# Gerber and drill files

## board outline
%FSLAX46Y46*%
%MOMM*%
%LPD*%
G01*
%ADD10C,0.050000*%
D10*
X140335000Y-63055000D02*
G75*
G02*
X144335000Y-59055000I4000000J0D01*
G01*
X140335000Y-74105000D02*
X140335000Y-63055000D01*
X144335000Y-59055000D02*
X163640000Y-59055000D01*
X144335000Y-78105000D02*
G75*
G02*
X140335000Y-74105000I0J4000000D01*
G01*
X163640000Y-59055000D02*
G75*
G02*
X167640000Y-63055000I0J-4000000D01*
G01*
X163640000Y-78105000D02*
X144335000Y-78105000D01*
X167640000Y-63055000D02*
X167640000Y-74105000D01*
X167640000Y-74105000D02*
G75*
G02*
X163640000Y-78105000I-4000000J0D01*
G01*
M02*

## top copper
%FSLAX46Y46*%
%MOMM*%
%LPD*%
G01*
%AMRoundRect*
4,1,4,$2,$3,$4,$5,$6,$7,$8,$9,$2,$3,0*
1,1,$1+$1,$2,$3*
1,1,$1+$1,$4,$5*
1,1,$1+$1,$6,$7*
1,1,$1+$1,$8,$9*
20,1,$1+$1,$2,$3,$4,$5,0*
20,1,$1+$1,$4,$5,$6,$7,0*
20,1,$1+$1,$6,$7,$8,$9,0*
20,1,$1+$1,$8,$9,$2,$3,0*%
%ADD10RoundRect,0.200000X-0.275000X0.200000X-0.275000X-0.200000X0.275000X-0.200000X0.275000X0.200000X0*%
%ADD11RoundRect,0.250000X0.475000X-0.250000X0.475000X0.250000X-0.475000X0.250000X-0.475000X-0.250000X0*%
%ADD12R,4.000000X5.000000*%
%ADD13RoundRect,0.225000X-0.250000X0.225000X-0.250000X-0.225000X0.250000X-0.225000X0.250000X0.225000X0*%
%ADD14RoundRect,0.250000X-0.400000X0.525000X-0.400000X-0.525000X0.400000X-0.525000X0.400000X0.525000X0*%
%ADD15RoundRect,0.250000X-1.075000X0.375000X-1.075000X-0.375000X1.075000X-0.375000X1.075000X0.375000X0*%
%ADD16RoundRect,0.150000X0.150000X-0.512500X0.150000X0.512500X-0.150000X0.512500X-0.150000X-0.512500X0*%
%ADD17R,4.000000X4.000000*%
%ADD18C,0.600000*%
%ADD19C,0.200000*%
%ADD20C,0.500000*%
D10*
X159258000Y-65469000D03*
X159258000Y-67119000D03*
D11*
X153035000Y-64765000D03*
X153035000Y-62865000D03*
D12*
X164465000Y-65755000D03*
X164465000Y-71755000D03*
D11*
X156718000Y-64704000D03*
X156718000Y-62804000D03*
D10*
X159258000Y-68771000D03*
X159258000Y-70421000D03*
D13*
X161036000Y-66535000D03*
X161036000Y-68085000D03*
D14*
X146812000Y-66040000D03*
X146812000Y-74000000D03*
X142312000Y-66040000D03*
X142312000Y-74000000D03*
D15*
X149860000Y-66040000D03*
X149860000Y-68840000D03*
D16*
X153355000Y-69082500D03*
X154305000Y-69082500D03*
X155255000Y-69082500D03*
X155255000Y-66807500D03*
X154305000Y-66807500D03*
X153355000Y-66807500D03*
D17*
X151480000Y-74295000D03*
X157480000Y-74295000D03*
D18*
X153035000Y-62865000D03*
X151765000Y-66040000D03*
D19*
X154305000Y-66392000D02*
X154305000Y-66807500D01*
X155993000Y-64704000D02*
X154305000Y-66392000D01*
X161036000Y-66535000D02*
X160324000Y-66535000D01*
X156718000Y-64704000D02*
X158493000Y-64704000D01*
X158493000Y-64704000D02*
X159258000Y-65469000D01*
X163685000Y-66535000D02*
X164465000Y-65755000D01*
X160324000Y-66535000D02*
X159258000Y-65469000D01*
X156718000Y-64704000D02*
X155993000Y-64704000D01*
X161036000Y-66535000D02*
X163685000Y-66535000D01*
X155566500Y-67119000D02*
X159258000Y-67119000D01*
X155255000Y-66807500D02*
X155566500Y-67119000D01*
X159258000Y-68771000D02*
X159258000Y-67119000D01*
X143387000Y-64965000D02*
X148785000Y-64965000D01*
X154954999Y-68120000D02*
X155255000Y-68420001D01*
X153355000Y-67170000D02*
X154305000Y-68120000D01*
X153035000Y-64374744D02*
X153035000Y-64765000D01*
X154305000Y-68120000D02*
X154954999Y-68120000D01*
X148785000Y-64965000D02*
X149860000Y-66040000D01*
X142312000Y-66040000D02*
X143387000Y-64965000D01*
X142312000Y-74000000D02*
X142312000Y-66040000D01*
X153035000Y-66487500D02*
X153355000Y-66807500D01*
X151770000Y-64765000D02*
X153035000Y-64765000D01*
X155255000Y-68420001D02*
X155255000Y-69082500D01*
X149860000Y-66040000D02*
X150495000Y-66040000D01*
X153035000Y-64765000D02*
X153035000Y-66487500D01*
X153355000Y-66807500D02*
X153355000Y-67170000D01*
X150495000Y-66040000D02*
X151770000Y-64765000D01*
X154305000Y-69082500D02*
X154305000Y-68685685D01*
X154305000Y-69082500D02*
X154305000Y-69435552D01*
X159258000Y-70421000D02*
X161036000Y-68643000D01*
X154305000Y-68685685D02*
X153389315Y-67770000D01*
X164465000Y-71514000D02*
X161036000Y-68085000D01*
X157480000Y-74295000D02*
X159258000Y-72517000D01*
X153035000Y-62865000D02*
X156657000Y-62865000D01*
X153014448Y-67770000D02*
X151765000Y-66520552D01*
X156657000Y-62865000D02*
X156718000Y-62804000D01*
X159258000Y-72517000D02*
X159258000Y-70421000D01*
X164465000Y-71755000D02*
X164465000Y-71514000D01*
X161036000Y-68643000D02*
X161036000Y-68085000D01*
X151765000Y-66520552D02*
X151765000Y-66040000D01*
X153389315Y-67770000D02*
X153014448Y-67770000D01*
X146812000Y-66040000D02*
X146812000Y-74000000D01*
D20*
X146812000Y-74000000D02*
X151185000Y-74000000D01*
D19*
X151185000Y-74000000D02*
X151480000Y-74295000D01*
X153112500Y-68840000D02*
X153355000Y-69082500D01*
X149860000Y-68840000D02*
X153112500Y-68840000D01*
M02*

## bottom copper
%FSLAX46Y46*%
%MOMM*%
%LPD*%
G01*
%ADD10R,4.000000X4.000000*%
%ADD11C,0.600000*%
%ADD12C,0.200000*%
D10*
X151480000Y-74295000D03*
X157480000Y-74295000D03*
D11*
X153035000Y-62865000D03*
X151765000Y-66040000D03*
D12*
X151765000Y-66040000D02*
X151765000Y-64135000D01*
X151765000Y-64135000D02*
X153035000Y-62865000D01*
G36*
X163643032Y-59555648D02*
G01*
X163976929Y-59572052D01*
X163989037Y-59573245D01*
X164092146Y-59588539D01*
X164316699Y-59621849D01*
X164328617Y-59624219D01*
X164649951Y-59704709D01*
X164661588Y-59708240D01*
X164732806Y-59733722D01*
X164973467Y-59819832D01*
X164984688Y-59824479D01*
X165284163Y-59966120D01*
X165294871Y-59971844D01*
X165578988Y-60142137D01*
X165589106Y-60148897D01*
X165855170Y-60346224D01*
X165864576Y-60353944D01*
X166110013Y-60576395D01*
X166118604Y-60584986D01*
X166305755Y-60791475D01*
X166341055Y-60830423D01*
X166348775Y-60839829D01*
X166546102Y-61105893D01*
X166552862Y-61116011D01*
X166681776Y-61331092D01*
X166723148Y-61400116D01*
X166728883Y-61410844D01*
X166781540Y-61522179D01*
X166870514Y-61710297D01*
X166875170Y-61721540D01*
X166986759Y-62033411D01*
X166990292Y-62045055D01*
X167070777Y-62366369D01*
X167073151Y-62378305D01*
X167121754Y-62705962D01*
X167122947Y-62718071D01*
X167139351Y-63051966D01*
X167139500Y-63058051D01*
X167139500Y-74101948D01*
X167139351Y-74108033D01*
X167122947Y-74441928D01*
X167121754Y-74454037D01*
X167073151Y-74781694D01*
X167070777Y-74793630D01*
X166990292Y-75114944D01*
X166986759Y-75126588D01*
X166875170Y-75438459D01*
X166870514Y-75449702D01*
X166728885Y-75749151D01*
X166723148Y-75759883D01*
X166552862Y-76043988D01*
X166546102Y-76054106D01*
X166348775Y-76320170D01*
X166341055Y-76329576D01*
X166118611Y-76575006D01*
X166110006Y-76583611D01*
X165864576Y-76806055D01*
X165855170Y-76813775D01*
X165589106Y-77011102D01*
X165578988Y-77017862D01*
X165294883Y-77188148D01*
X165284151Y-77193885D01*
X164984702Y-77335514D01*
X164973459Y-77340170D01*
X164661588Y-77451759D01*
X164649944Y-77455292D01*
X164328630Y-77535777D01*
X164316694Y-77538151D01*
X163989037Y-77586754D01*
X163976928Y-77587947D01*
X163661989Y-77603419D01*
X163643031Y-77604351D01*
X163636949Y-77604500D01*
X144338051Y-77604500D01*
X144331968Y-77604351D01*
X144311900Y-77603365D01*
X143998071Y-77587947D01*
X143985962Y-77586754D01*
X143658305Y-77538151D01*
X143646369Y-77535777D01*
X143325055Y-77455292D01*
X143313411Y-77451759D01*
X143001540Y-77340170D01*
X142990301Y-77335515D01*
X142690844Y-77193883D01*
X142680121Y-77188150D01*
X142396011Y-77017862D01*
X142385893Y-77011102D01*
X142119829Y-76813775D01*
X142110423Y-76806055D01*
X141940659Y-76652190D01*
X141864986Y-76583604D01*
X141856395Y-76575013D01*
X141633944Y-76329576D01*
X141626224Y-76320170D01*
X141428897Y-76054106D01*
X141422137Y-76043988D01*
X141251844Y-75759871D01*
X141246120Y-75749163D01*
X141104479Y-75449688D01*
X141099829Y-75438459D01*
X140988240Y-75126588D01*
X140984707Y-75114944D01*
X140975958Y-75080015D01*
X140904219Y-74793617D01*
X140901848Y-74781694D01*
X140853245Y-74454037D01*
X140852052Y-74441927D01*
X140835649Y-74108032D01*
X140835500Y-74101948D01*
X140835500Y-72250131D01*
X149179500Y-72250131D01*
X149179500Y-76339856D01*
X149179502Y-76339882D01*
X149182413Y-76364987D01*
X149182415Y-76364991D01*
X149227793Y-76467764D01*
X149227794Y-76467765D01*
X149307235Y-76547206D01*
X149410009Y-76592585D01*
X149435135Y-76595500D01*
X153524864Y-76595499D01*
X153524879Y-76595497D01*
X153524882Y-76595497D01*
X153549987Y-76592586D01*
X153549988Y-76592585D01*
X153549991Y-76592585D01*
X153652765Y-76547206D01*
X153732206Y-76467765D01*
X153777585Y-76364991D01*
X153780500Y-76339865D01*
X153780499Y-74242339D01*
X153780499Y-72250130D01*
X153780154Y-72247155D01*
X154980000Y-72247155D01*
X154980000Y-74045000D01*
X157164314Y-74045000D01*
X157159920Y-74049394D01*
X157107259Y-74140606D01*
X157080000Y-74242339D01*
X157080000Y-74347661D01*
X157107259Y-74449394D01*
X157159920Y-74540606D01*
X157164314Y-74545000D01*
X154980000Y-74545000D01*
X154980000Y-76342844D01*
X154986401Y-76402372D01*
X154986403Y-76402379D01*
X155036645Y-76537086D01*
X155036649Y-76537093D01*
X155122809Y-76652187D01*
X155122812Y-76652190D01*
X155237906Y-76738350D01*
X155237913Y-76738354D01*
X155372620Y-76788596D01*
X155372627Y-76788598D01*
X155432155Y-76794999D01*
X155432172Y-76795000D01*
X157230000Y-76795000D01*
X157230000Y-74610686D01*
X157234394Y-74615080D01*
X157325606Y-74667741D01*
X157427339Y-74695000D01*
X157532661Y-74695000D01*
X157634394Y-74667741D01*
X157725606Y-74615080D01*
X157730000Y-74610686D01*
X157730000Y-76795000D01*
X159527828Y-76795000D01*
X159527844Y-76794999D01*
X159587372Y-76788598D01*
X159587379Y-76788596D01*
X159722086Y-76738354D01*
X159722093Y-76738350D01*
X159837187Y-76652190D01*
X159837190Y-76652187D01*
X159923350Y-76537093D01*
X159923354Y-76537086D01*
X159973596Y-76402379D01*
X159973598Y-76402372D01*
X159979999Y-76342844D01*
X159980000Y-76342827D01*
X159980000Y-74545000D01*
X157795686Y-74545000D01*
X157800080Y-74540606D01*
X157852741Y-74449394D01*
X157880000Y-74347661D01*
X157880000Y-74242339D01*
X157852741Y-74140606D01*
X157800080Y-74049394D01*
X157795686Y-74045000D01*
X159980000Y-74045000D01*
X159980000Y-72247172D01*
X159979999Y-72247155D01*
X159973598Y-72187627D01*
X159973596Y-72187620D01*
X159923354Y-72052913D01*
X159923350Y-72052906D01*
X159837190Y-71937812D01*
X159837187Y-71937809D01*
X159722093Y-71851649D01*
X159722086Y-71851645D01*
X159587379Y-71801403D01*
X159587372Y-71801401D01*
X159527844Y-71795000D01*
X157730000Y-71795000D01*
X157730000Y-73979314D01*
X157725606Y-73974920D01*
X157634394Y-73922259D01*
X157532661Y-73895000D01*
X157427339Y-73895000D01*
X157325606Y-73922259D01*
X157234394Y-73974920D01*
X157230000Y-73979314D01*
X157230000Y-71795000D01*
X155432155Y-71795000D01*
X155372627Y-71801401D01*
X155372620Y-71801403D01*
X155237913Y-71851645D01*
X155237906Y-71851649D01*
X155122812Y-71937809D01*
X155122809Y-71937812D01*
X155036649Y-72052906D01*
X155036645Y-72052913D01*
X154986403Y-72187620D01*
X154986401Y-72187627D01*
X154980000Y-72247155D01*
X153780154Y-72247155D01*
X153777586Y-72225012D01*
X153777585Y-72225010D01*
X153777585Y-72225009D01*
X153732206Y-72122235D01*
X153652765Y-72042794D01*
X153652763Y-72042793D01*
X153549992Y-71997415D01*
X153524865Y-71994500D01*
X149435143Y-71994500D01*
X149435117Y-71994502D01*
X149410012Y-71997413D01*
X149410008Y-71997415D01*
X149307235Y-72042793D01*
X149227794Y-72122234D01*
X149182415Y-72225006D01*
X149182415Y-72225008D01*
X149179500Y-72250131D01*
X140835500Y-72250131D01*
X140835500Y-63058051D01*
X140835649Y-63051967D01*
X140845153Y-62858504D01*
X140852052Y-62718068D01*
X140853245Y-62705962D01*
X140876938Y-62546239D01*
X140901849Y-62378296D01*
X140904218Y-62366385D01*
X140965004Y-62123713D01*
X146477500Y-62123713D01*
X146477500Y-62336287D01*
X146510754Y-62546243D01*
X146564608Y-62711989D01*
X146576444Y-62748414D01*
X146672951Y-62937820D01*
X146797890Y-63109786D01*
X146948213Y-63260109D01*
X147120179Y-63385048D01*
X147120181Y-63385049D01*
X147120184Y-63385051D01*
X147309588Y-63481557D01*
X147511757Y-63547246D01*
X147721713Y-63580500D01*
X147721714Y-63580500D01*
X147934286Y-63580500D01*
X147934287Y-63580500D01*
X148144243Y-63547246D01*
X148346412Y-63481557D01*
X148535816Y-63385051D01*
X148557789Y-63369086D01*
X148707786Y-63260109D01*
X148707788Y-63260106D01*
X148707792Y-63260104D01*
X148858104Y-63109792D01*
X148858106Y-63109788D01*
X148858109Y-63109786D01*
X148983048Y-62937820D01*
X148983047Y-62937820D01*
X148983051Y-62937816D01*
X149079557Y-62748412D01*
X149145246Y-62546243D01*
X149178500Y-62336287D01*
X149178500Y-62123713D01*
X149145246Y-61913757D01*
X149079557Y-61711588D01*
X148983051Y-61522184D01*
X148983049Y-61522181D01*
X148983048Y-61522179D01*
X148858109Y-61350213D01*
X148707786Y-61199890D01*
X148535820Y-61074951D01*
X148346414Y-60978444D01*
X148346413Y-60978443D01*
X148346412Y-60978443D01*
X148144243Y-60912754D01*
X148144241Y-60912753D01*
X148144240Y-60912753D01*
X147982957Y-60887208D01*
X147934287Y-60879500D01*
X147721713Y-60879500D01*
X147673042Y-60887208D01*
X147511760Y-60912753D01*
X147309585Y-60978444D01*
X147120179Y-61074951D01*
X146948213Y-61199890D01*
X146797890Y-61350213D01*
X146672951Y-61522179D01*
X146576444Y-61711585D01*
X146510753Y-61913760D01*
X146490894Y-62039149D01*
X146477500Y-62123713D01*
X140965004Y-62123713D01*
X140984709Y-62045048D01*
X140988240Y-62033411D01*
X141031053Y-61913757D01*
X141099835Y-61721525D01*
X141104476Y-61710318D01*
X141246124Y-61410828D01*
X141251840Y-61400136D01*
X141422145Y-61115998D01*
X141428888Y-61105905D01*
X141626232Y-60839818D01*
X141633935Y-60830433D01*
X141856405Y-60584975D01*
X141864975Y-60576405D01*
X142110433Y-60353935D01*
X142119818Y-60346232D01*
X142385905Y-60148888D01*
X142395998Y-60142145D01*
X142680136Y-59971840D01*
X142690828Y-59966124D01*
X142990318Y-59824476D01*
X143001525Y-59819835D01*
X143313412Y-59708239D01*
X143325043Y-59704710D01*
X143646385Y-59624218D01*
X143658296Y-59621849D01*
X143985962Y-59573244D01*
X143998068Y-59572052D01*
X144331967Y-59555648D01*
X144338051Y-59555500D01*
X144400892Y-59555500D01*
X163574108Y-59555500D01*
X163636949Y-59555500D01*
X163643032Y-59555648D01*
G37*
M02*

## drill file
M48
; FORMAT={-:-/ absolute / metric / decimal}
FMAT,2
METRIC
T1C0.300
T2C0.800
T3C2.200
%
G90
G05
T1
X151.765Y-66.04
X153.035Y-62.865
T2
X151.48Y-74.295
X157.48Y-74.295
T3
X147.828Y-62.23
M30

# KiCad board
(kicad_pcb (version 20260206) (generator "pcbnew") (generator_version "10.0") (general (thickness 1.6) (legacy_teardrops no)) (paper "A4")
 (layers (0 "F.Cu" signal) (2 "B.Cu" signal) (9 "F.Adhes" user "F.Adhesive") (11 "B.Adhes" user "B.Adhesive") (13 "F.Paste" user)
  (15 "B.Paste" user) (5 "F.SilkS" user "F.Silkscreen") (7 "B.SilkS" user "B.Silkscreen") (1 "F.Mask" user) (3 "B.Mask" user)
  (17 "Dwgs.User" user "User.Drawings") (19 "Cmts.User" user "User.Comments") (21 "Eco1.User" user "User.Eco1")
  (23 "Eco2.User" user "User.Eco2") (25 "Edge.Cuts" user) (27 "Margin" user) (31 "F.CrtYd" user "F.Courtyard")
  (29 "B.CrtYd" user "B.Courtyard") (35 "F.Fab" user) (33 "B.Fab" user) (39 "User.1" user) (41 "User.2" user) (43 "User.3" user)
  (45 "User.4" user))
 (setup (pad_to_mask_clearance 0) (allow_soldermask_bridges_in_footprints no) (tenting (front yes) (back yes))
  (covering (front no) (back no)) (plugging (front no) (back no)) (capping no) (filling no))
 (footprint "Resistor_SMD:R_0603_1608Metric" (layer "F.Cu") (at 159.258 66.294 -90)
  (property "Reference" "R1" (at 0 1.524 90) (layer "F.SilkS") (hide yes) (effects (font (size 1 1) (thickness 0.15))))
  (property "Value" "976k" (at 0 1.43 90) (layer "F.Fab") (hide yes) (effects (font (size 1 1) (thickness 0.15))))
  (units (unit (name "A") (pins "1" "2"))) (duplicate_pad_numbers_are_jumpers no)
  (pad "1" smd roundrect (at -0.825 0 270) (size 0.8 0.95) (layers "F.Cu" "F.Mask" "F.Paste") (roundrect_rratio 0.25) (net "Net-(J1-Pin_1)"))
  (pad "2" smd roundrect (at 0.825 0 270) (size 0.8 0.95) (layers "F.Cu" "F.Mask" "F.Paste") (roundrect_rratio 0.25) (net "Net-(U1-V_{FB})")))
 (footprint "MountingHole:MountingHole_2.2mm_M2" (layer "F.Cu") (at 147.828 62.23)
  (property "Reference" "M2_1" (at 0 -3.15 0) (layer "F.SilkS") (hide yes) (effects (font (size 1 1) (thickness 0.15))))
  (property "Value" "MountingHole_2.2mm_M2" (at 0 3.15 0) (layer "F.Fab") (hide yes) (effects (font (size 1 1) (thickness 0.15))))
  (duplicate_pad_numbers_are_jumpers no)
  (pad "" np_thru_hole circle (at 0 0) (size 2.2 2.2) (drill 2.2) (layers "*.Cu" "*.Mask")))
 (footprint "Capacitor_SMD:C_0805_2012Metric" (layer "F.Cu") (at 153.035 63.815 90)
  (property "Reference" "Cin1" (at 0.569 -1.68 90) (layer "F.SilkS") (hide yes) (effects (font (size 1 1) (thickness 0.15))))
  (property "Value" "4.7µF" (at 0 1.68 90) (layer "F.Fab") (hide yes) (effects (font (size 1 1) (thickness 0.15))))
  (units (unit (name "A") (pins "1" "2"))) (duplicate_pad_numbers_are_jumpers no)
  (pad "1" smd roundrect (at -0.95 0 90) (size 1 1.45) (layers "F.Cu" "F.Mask" "F.Paste") (roundrect_rratio 0.25) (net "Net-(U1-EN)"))
  (pad "2" smd roundrect (at 0.95 0 90) (size 1 1.45) (layers "F.Cu" "F.Mask" "F.Paste") (roundrect_rratio 0.25) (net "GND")))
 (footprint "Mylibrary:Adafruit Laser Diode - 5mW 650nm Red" (layer "F.Cu") (at 164.465 68.755 -90)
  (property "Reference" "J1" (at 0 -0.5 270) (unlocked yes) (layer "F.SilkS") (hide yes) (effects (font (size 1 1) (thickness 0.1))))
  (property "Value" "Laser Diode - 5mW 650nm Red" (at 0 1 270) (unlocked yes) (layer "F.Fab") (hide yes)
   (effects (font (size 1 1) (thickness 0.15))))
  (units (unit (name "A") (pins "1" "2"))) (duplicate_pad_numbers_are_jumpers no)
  (pad "1" smd rect (at -3 0 270) (size 5 4) (layers "F.Cu" "F.Mask" "F.Paste") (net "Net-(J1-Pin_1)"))
  (pad "2" smd rect (at 3 0 270) (size 5 4) (layers "F.Cu" "F.Mask" "F.Paste") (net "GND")))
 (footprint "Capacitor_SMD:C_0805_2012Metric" (layer "F.Cu") (at 156.718 63.754 90)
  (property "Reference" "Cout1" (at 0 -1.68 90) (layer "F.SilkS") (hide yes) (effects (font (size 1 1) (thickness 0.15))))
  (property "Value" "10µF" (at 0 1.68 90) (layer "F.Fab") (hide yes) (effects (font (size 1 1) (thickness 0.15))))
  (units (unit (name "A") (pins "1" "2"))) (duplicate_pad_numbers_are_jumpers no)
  (pad "1" smd roundrect (at -0.95 0 90) (size 1 1.45) (layers "F.Cu" "F.Mask" "F.Paste") (roundrect_rratio 0.25) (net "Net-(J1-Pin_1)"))
  (pad "2" smd roundrect (at 0.95 0 90) (size 1 1.45) (layers "F.Cu" "F.Mask" "F.Paste") (roundrect_rratio 0.25) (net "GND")))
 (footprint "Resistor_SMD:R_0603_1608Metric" (layer "F.Cu") (at 159.258 69.596 -90)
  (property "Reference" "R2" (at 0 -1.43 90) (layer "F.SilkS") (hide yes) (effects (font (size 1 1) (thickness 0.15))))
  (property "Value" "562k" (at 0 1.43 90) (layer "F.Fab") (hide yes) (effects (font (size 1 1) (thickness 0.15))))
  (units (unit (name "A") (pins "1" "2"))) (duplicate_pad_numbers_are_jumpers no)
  (pad "1" smd roundrect (at -0.825 0 270) (size 0.8 0.95) (layers "F.Cu" "F.Mask" "F.Paste") (roundrect_rratio 0.25)
   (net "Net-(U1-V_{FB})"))
  (pad "2" smd roundrect (at 0.825 0 270) (size 0.8 0.95) (layers "F.Cu" "F.Mask" "F.Paste") (roundrect_rratio 0.25) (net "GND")))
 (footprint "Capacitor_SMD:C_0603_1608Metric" (layer "F.Cu") (at 161.036 67.31 -90)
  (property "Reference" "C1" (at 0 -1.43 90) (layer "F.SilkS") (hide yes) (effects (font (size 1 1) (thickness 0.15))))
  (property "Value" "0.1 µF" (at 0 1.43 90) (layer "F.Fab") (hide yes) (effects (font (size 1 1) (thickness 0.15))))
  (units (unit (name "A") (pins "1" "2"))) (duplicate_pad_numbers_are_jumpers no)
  (pad "1" smd roundrect (at -0.775 0 270) (size 0.9 0.95) (layers "F.Cu" "F.Mask" "F.Paste") (roundrect_rratio 0.25) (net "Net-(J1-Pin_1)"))
  (pad "2" smd roundrect (at 0.775 0 270) (size 0.9 0.95) (layers "F.Cu" "F.Mask" "F.Paste") (roundrect_rratio 0.25) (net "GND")))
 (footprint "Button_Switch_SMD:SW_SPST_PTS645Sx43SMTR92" (layer "F.Cu") (at 144.562 70.02 -90)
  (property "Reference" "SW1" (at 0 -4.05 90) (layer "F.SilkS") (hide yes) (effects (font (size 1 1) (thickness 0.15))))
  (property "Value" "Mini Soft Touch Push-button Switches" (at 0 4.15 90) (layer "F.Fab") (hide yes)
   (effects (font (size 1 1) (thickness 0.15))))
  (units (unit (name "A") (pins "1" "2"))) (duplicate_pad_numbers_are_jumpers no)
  (pad "1" smd roundrect (at -3.98 -2.25 270) (size 1.55 1.3) (layers "F.Cu" "F.Mask" "F.Paste") (roundrect_rratio 0.1923076923)
   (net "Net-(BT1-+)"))
  (pad "1" smd roundrect (at 3.98 -2.25 270) (size 1.55 1.3) (layers "F.Cu" "F.Mask" "F.Paste") (roundrect_rratio 0.1923076923)
   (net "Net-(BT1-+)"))
  (pad "2" smd roundrect (at -3.98 2.25 270) (size 1.55 1.3) (layers "F.Cu" "F.Mask" "F.Paste") (roundrect_rratio 0.1923076923)
   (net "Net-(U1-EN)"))
  (pad "2" smd roundrect (at 3.98 2.25 270) (size 1.55 1.3) (layers "F.Cu" "F.Mask" "F.Paste") (roundrect_rratio 0.1923076923)
   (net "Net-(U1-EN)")))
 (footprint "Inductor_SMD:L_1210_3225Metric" (layer "F.Cu") (at 149.86 67.44 -90)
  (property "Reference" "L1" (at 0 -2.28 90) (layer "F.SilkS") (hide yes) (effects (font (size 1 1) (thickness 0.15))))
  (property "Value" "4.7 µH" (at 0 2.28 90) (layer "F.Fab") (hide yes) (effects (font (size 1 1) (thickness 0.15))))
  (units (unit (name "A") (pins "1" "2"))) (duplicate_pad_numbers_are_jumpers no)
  (pad "1" smd roundrect (at -1.4 0 270) (size 1.25 2.65) (layers "F.Cu" "F.Mask" "F.Paste") (roundrect_rratio 0.2) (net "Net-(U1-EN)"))
  (pad "2" smd roundrect (at 1.4 0 270) (size 1.25 2.65) (layers "F.Cu" "F.Mask" "F.Paste") (roundrect_rratio 0.2) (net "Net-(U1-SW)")))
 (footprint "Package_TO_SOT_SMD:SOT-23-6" (layer "F.Cu") (at 154.305 67.945 90)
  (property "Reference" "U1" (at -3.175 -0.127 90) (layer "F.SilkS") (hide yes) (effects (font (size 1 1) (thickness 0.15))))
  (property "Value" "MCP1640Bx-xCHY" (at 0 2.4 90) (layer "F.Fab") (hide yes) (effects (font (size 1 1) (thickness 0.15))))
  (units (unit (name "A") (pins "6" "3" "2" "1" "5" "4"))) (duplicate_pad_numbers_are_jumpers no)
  (pad "1" smd roundrect (at -1.1375 -0.95 90) (size 1.325 0.6) (layers "F.Cu" "F.Mask" "F.Paste") (roundrect_rratio 0.25)
   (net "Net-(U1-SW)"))
  (pad "2" smd roundrect (at -1.1375 0 90) (size 1.325 0.6) (layers "F.Cu" "F.Mask" "F.Paste") (roundrect_rratio 0.25) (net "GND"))
  (pad "3" smd roundrect (at -1.1375 0.95 90) (size 1.325 0.6) (layers "F.Cu" "F.Mask" "F.Paste") (roundrect_rratio 0.25)
   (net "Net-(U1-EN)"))
  (pad "4" smd roundrect (at 1.1375 0.95 90) (size 1.325 0.6) (layers "F.Cu" "F.Mask" "F.Paste") (roundrect_rratio 0.25)
   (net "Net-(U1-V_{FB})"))
  (pad "5" smd roundrect (at 1.1375 0 90) (size 1.325 0.6) (layers "F.Cu" "F.Mask" "F.Paste") (roundrect_rratio 0.25) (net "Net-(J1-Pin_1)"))
  (pad "6" smd roundrect (at 1.1375 -0.95 90) (size 1.325 0.6) (layers "F.Cu" "F.Mask" "F.Paste") (roundrect_rratio 0.25)
   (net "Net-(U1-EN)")))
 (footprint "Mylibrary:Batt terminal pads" (layer "F.Cu") (at 151.48 74.295)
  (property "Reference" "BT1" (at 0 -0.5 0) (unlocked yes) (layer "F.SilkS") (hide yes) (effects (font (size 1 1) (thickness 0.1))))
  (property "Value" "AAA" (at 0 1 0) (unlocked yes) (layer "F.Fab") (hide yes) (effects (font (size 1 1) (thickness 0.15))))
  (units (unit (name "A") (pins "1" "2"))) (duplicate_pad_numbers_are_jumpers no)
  (pad "1" thru_hole rect (at 0 0) (size 4 4) (drill 0.8) (layers "*.Cu" "*.Mask") (remove_unused_layers no) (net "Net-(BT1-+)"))
  (pad "2" thru_hole rect (at 6 0) (size 4 4) (drill 0.8) (layers "*.Cu" "*.Mask") (remove_unused_layers no) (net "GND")))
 (gr_arc (start 140.335 63.055) (mid 141.506573 60.226573) (end 144.335 59.055) (stroke (width 0.05) (type default)) (layer "Edge.Cuts"))
 (gr_line (start 140.335 74.105) (end 140.335 63.055) (stroke (width 0.05) (type default)) (layer "Edge.Cuts"))
 (gr_line (start 144.335 59.055) (end 163.64 59.055) (stroke (width 0.05) (type default)) (layer "Edge.Cuts"))
 (gr_arc (start 144.335 78.105) (mid 141.506573 76.933427) (end 140.335 74.105) (stroke (width 0.05) (type default)) (layer "Edge.Cuts"))
 (gr_arc (start 163.64 59.055) (mid 166.468427 60.226573) (end 167.64 63.055) (stroke (width 0.05) (type default)) (layer "Edge.Cuts"))
 (gr_line (start 163.64 78.105) (end 144.335 78.105) (stroke (width 0.05) (type default)) (layer "Edge.Cuts"))
 (gr_line (start 167.64 63.055) (end 167.64 74.105) (stroke (width 0.05) (type default)) (layer "Edge.Cuts"))
 (gr_arc (start 167.64 74.105) (mid 166.468427 76.933427) (end 163.64 78.105) (stroke (width 0.05) (type default)) (layer "Edge.Cuts"))
 (segment (start 154.305 66.392) (end 154.305 66.8075) (width 0.2) (layer "F.Cu") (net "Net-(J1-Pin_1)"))
 (segment (start 155.993 64.704) (end 154.305 66.392) (width 0.2) (layer "F.Cu") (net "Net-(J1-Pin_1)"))
 (segment (start 161.036 66.535) (end 160.324 66.535) (width 0.2) (layer "F.Cu") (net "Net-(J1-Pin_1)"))
 (segment (start 156.718 64.704) (end 158.493 64.704) (width 0.2) (layer "F.Cu") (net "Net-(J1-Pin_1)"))
 (segment (start 158.493 64.704) (end 159.258 65.469) (width 0.2) (layer "F.Cu") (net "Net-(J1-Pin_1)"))
 (segment (start 163.685 66.535) (end 164.465 65.755) (width 0.2) (layer "F.Cu") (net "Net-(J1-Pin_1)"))
 (segment (start 160.324 66.535) (end 159.258 65.469) (width 0.2) (layer "F.Cu") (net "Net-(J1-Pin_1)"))
 (segment (start 156.718 64.704) (end 155.993 64.704) (width 0.2) (layer "F.Cu") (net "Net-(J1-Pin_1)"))
 (segment (start 161.036 66.535) (end 163.685 66.535) (width 0.2) (layer "F.Cu") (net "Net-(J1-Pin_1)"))
 (segment (start 155.5665 67.119) (end 159.258 67.119) (width 0.2) (layer "F.Cu") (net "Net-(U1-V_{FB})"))
 (segment (start 155.255 66.8075) (end 155.5665 67.119) (width 0.2) (layer "F.Cu") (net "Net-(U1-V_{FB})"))
 (segment (start 159.258 68.771) (end 159.258 67.119) (width 0.2) (layer "F.Cu") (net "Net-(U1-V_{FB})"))
 (segment (start 143.387 64.965) (end 148.785 64.965) (width 0.2) (layer "F.Cu") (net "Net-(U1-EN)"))
 (segment (start 154.954999 68.12) (end 155.255 68.420001) (width 0.2) (layer "F.Cu") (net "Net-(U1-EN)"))
 (segment (start 153.355 67.17) (end 154.305 68.12) (width 0.2) (layer "F.Cu") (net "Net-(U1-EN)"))
 (segment (start 153.035 64.374744) (end 153.035 64.765) (width 0.2) (layer "F.Cu") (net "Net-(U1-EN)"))
 (segment (start 154.305 68.12) (end 154.954999 68.12) (width 0.2) (layer "F.Cu") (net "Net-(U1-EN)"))
 (segment (start 148.785 64.965) (end 149.86 66.04) (width 0.2) (layer "F.Cu") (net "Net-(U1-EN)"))
 (segment (start 142.312 66.04) (end 143.387 64.965) (width 0.2) (layer "F.Cu") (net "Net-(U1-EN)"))
 (segment (start 142.312 74) (end 142.312 66.04) (width 0.2) (layer "F.Cu") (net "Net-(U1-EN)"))
 (segment (start 153.035 66.4875) (end 153.355 66.8075) (width 0.2) (layer "F.Cu") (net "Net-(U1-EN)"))
 (segment (start 151.77 64.765) (end 153.035 64.765) (width 0.2) (layer "F.Cu") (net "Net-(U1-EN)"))
 (segment (start 155.255 68.420001) (end 155.255 69.0825) (width 0.2) (layer "F.Cu") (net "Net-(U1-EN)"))
 (segment (start 149.86 66.04) (end 150.495 66.04) (width 0.2) (layer "F.Cu") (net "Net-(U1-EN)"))
 (segment (start 153.035 64.765) (end 153.035 66.4875) (width 0.2) (layer "F.Cu") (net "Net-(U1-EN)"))
 (segment (start 153.355 66.8075) (end 153.355 67.17) (width 0.2) (layer "F.Cu") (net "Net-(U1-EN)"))
 (segment (start 150.495 66.04) (end 151.77 64.765) (width 0.2) (layer "F.Cu") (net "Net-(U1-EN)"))
 (segment (start 154.305 69.0825) (end 154.305 68.685685) (width 0.2) (layer "F.Cu") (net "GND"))
 (segment (start 154.305 69.0825) (end 154.305 69.435552) (width 0.2) (layer "F.Cu") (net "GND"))
 (segment (start 159.258 70.421) (end 161.036 68.643) (width 0.2) (layer "F.Cu") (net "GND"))
 (segment (start 154.305 68.685685) (end 153.389315 67.77) (width 0.2) (layer "F.Cu") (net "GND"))
 (segment (start 164.465 71.514) (end 161.036 68.085) (width 0.2) (layer "F.Cu") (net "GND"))
 (segment (start 157.48 74.295) (end 159.258 72.517) (width 0.2) (layer "F.Cu") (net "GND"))
 (segment (start 153.035 62.865) (end 156.657 62.865) (width 0.2) (layer "F.Cu") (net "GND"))
 (segment (start 153.014448 67.77) (end 151.765 66.520552) (width 0.2) (layer "F.Cu") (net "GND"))
 (segment (start 156.657 62.865) (end 156.718 62.804) (width 0.2) (layer "F.Cu") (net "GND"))
 (segment (start 159.258 72.517) (end 159.258 70.421) (width 0.2) (layer "F.Cu") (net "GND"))
 (segment (start 164.465 71.755) (end 164.465 71.514) (width 0.2) (layer "F.Cu") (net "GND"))
 (segment (start 161.036 68.643) (end 161.036 68.085) (width 0.2) (layer "F.Cu") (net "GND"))
 (segment (start 151.765 66.520552) (end 151.765 66.04) (width 0.2) (layer "F.Cu") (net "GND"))
 (segment (start 153.389315 67.77) (end 153.014448 67.77) (width 0.2) (layer "F.Cu") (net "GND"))
 (via (at 153.035 62.865) (size 0.6) (drill 0.3) (layers "F.Cu" "B.Cu") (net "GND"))
 (via (at 151.765 66.04) (size 0.6) (drill 0.3) (layers "F.Cu" "B.Cu") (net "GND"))
 (segment (start 151.765 66.04) (end 151.765 64.135) (width 0.2) (layer "B.Cu") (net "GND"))
 (segment (start 151.765 64.135) (end 153.035 62.865) (width 0.2) (layer "B.Cu") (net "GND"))
 (segment (start 146.812 66.04) (end 146.812 74) (width 0.2) (layer "F.Cu") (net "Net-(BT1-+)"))
 (segment (start 146.812 74) (end 151.185 74) (width 0.5) (layer "F.Cu") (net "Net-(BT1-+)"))
 (segment (start 151.185 74) (end 151.48 74.295) (width 0.2) (layer "F.Cu") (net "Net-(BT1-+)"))
 (segment (start 153.1125 68.84) (end 153.355 69.0825) (width 0.2) (layer "F.Cu") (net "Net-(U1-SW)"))
 (segment (start 149.86 68.84) (end 153.1125 68.84) (width 0.2) (layer "F.Cu") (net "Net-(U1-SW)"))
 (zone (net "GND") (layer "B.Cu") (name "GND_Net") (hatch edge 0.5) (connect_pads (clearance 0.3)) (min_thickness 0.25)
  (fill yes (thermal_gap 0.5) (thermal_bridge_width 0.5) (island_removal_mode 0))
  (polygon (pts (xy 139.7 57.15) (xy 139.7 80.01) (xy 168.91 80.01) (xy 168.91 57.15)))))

